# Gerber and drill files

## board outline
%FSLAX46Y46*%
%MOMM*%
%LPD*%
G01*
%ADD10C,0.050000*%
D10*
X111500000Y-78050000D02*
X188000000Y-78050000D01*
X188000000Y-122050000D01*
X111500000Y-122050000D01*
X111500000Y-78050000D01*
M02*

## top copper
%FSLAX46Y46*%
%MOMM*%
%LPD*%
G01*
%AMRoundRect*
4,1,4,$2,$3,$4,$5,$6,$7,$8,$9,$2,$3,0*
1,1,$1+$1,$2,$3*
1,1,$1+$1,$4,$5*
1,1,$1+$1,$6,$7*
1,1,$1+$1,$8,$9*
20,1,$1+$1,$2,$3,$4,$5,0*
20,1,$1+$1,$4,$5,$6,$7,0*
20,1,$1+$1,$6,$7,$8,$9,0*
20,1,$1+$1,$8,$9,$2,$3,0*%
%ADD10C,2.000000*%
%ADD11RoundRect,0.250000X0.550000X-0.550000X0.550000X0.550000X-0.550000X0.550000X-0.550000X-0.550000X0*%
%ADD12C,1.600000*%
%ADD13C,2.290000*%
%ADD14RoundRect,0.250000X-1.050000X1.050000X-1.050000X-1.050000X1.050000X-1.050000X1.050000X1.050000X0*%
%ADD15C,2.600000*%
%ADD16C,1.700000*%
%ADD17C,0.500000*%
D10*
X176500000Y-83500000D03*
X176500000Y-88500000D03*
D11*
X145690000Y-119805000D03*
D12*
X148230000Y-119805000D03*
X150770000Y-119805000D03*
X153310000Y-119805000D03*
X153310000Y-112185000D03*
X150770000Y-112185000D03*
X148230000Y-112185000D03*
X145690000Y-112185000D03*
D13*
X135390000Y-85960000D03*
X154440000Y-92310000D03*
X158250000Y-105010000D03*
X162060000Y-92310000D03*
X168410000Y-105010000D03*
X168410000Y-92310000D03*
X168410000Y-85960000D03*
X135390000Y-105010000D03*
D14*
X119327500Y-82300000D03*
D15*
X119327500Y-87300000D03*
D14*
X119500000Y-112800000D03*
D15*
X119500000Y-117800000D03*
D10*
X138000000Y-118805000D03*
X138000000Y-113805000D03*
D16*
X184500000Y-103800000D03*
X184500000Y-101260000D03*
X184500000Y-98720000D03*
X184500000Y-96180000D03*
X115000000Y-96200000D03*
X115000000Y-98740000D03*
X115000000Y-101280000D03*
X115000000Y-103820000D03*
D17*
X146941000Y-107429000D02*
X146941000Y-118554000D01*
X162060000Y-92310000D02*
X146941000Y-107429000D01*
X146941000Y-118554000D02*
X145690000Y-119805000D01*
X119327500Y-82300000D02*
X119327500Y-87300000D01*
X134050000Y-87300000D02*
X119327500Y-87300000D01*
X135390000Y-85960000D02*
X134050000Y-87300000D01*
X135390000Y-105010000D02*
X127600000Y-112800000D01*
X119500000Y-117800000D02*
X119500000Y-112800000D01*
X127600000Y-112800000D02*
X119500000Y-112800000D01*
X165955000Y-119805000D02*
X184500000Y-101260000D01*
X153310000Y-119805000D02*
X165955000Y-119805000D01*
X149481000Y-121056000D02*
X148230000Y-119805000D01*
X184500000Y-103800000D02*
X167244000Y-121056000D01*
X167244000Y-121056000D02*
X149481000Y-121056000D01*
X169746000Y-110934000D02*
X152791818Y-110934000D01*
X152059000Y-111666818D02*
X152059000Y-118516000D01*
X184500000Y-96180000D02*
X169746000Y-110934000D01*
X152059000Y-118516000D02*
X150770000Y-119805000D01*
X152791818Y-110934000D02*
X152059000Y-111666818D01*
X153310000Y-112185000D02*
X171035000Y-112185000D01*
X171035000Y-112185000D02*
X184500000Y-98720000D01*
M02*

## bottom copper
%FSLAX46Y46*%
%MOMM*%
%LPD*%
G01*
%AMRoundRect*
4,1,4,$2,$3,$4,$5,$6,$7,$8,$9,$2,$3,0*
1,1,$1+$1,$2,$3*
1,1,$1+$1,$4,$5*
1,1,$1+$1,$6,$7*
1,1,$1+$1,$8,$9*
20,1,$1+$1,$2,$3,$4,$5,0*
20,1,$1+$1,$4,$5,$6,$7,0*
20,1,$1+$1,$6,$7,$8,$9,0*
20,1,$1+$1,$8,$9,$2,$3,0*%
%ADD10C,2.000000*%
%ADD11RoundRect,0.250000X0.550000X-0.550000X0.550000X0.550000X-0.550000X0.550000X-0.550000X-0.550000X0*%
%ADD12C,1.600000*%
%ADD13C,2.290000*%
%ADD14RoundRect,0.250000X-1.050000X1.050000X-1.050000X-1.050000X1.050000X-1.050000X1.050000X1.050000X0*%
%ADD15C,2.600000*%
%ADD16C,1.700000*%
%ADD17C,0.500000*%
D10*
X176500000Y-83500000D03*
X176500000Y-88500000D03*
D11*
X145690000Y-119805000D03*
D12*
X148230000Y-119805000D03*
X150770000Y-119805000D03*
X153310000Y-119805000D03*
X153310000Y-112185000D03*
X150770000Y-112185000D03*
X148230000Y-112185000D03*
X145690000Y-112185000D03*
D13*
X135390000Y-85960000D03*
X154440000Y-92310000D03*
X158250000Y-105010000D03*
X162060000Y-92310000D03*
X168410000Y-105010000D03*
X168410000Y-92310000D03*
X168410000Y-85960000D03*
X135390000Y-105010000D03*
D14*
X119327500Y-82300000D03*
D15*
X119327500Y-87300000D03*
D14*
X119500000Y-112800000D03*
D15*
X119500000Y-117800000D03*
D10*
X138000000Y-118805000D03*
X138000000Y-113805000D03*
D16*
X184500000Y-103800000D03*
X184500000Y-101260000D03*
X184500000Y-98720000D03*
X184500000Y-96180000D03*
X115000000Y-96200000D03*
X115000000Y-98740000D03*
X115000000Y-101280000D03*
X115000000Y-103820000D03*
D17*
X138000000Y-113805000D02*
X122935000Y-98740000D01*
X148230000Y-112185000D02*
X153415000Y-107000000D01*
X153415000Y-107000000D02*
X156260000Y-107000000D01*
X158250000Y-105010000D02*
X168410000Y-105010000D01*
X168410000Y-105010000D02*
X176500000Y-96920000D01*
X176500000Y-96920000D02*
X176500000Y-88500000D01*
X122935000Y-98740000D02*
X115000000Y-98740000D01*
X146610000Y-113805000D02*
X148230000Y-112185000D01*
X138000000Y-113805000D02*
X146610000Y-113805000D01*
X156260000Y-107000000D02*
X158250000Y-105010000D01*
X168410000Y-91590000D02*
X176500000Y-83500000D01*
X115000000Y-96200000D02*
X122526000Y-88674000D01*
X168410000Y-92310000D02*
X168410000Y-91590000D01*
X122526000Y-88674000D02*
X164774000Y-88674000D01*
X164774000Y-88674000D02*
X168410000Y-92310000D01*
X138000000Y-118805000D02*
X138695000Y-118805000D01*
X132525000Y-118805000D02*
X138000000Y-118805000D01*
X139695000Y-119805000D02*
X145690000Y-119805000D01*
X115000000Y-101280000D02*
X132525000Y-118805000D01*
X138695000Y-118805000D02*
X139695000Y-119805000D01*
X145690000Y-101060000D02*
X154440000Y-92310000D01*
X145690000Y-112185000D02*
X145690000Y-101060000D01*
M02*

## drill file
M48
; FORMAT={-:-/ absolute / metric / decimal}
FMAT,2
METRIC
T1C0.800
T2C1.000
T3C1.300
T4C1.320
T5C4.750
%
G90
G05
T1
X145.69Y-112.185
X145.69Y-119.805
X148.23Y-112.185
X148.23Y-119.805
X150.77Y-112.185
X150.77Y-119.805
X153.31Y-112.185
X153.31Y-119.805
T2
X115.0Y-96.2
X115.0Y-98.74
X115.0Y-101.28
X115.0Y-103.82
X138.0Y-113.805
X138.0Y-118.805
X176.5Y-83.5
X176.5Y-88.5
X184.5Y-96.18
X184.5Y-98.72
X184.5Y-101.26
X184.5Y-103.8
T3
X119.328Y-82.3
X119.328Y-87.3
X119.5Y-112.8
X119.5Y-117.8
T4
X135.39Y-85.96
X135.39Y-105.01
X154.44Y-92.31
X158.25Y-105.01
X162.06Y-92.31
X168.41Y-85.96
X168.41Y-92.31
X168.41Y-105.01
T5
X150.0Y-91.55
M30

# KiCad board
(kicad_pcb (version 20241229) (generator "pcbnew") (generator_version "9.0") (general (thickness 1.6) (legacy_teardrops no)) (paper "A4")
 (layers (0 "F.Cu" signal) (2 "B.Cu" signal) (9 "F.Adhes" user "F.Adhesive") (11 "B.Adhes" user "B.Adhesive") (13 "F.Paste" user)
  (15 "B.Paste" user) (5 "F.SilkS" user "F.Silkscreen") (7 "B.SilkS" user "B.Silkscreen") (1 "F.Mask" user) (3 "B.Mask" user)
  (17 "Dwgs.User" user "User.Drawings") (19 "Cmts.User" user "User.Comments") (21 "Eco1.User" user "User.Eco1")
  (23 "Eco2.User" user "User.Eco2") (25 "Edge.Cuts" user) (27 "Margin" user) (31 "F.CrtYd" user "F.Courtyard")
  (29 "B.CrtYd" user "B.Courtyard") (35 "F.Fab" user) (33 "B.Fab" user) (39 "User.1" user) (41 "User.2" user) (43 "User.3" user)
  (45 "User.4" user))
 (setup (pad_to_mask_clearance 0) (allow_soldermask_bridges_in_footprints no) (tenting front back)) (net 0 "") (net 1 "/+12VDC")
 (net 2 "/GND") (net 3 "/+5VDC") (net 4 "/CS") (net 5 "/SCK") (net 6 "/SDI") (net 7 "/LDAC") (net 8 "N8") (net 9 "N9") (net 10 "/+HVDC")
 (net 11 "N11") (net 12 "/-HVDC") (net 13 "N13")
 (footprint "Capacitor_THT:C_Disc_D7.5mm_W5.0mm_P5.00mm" (layer "F.Cu") (at 176.5 83.5 -90)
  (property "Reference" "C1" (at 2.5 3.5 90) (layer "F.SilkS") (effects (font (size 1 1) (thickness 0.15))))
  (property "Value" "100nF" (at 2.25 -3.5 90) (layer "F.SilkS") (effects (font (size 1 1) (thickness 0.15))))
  (pad "1" thru_hole circle (at 0 0 270) (size 2 2) (drill 1) (layers "*.Cu" "*.Mask") (remove_unused_layers no) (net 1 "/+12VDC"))
  (pad "2" thru_hole circle (at 5 0 270) (size 2 2) (drill 1) (layers "*.Cu" "*.Mask") (remove_unused_layers no) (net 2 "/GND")))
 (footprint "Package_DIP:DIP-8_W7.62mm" (layer "F.Cu") (at 145.69 119.805 90)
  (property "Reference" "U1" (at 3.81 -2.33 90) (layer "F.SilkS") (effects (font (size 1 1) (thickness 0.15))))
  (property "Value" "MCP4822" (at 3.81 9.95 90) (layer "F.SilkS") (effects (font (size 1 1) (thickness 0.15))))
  (pad "1" thru_hole roundrect (at 0 0 90) (size 1.6 1.6) (drill 0.8) (layers "*.Cu" "*.Mask") (remove_unused_layers no)
   (roundrect_rratio 0.15625) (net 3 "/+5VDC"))
  (pad "2" thru_hole circle (at 0 2.54 90) (size 1.6 1.6) (drill 0.8) (layers "*.Cu" "*.Mask") (remove_unused_layers no) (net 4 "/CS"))
  (pad "3" thru_hole circle (at 0 5.08 90) (size 1.6 1.6) (drill 0.8) (layers "*.Cu" "*.Mask") (remove_unused_layers no) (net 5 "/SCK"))
  (pad "4" thru_hole circle (at 0 7.62 90) (size 1.6 1.6) (drill 0.8) (layers "*.Cu" "*.Mask") (remove_unused_layers no) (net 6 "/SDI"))
  (pad "5" thru_hole circle (at 7.62 7.62 90) (size 1.6 1.6) (drill 0.8) (layers "*.Cu" "*.Mask") (remove_unused_layers no) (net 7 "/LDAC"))
  (pad "6" thru_hole circle (at 7.62 5.08 90) (size 1.6 1.6) (drill 0.8) (layers "*.Cu" "*.Mask") (remove_unused_layers no) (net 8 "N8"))
  (pad "7" thru_hole circle (at 7.62 2.54 90) (size 1.6 1.6) (drill 0.8) (layers "*.Cu" "*.Mask") (remove_unused_layers no) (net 2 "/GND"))
  (pad "8" thru_hole circle (at 7.62 0 90) (size 1.6 1.6) (drill 0.8) (layers "*.Cu" "*.Mask") (remove_unused_layers no) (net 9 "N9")))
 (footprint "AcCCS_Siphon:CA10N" (layer "F.Cu") (at 135.39 85.96)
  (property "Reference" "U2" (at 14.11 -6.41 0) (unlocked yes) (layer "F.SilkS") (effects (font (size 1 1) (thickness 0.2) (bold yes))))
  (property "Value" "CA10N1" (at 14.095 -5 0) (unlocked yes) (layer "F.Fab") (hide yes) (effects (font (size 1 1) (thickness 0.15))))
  (pad "" np_thru_hole circle (at 14.61 5.59) (size 4.75 4.75) (drill 4.75) (layers "*.Cu" "*.Mask"))
  (pad "1" thru_hole circle (at 0 0) (size 2.29 2.29) (drill 1.32) (layers "*.Cu" "*.Mask") (remove_unused_layers no) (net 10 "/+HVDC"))
  (pad "2" thru_hole circle (at 19.05 6.35) (size 2.29 2.29) (drill 1.32) (layers "*.Cu" "*.Mask") (remove_unused_layers no) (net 9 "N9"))
  (pad "3" thru_hole circle (at 22.86 19.05) (size 2.29 2.29) (drill 1.32) (layers "*.Cu" "*.Mask") (remove_unused_layers no) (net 2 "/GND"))
  (pad "4" thru_hole circle (at 26.67 6.35) (size 2.29 2.29) (drill 1.32) (layers "*.Cu" "*.Mask") (remove_unused_layers no)
   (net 3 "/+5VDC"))
  (pad "5" thru_hole circle (at 33.02 19.05) (size 2.29 2.29) (drill 1.32) (layers "*.Cu" "*.Mask") (remove_unused_layers no) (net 2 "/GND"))
  (pad "6" thru_hole circle (at 33.02 6.35) (size 2.29 2.29) (drill 1.32) (layers "*.Cu" "*.Mask") (remove_unused_layers no)
   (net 1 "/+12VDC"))
  (pad "7" thru_hole circle (at 33.02 0) (size 2.29 2.29) (drill 1.32) (layers "*.Cu" "*.Mask") (remove_unused_layers no) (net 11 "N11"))
  (pad "8" thru_hole circle (at 0 19.05) (size 2.29 2.29) (drill 1.32) (layers "*.Cu" "*.Mask") (remove_unused_layers no) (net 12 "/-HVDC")))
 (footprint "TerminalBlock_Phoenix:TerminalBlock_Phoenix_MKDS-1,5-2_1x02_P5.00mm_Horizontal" (layer "F.Cu") (at 119.3275 82.3 -90)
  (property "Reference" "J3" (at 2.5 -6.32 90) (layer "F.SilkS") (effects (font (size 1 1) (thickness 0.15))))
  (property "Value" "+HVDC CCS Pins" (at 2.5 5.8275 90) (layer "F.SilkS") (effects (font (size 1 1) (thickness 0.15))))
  (pad "1" thru_hole roundrect (at 0 0 270) (size 2.6 2.6) (drill 1.3) (layers "*.Cu" "*.Mask") (remove_unused_layers no)
   (roundrect_rratio 0.096154) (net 10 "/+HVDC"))
  (pad "2" thru_hole circle (at 5 0 270) (size 2.6 2.6) (drill 1.3) (layers "*.Cu" "*.Mask") (remove_unused_layers no) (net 10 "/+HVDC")))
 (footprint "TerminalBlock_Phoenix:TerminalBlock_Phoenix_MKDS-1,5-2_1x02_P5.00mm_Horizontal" (layer "F.Cu") (at 119.5 112.8 -90)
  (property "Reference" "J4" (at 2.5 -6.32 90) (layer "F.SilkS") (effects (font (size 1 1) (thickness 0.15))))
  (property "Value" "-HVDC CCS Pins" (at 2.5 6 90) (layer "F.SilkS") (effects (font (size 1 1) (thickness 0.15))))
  (pad "1" thru_hole roundrect (at 0 0 270) (size 2.6 2.6) (drill 1.3) (layers "*.Cu" "*.Mask") (remove_unused_layers no)
   (roundrect_rratio 0.096154) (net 12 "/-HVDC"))
  (pad "2" thru_hole circle (at 5 0 270) (size 2.6 2.6) (drill 1.3) (layers "*.Cu" "*.Mask") (remove_unused_layers no) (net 12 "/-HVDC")))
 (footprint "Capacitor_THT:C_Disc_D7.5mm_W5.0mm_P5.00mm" (layer "F.Cu") (at 138 118.805 90)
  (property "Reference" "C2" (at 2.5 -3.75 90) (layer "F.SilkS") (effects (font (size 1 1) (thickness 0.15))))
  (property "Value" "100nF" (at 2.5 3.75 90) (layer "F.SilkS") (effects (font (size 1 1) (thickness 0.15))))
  (pad "1" thru_hole circle (at 0 0 90) (size 2 2) (drill 1) (layers "*.Cu" "*.Mask") (remove_unused_layers no) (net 3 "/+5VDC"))
  (pad "2" thru_hole circle (at 5 0 90) (size 2 2) (drill 1) (layers "*.Cu" "*.Mask") (remove_unused_layers no) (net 2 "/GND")))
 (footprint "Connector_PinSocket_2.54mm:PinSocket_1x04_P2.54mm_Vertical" (layer "B.Cu") (at 184.5 103.8)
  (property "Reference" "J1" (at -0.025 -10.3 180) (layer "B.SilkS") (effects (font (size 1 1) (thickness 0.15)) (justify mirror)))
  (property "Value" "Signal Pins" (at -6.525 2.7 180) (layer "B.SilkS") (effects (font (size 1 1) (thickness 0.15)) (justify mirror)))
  (pad "1" thru_hole circle (at 0 0) (size 1.7 1.7) (drill 1) (layers "*.Cu" "*.Mask") (remove_unused_layers no) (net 4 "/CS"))
  (pad "2" thru_hole circle (at 0 -2.54) (size 1.7 1.7) (drill 1) (layers "*.Cu" "*.Mask") (remove_unused_layers no) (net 6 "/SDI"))
  (pad "3" thru_hole circle (at 0 -5.08) (size 1.7 1.7) (drill 1) (layers "*.Cu" "*.Mask") (remove_unused_layers no) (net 7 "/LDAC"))
  (pad "4" thru_hole circle (at 0 -7.62) (size 1.7 1.7) (drill 1) (layers "*.Cu" "*.Mask") (remove_unused_layers no) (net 5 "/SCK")))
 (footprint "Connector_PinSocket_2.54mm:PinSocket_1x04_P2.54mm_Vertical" (layer "B.Cu") (at 115 96.2 180)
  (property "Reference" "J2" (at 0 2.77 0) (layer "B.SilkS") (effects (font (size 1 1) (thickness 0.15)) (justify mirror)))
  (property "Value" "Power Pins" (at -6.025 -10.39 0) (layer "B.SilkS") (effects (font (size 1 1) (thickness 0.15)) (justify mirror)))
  (pad "1" thru_hole circle (at 0 0 180) (size 1.7 1.7) (drill 1) (layers "*.Cu" "*.Mask") (remove_unused_layers no) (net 1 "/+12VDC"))
  (pad "2" thru_hole circle (at 0 -2.54 180) (size 1.7 1.7) (drill 1) (layers "*.Cu" "*.Mask") (remove_unused_layers no) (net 2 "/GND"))
  (pad "3" thru_hole circle (at 0 -5.08 180) (size 1.7 1.7) (drill 1) (layers "*.Cu" "*.Mask") (remove_unused_layers no) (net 3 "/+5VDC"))
  (pad "4" thru_hole circle (at 0 -7.62 180) (size 1.7 1.7) (drill 1) (layers "*.Cu" "*.Mask") (remove_unused_layers no) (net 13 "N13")))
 (gr_rect (start 111.5 78.05) (end 188 122.05) (stroke (width 0.05) (type default)) (fill no) (layer "Edge.Cuts"))
 (segment (start 138 113.805) (end 122.935 98.74) (width 0.5) (layer "B.Cu") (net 2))
 (segment (start 148.23 112.185) (end 153.415 107) (width 0.5) (layer "B.Cu") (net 2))
 (segment (start 153.415 107) (end 156.26 107) (width 0.5) (layer "B.Cu") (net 2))
 (segment (start 158.25 105.01) (end 168.41 105.01) (width 0.5) (layer "B.Cu") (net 2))
 (segment (start 168.41 105.01) (end 176.5 96.92) (width 0.5) (layer "B.Cu") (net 2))
 (segment (start 176.5 96.92) (end 176.5 88.5) (width 0.5) (layer "B.Cu") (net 2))
 (segment (start 122.935 98.74) (end 115 98.74) (width 0.5) (layer "B.Cu") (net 2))
 (segment (start 146.61 113.805) (end 148.23 112.185) (width 0.5) (layer "B.Cu") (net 2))
 (segment (start 138 113.805) (end 146.61 113.805) (width 0.5) (layer "B.Cu") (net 2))
 (segment (start 156.26 107) (end 158.25 105.01) (width 0.5) (layer "B.Cu") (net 2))
 (segment (start 168.41 91.59) (end 176.5 83.5) (width 0.5) (layer "B.Cu") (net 1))
 (segment (start 115 96.2) (end 122.526 88.674) (width 0.5) (layer "B.Cu") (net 1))
 (segment (start 168.41 92.31) (end 168.41 91.59) (width 0.5) (layer "B.Cu") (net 1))
 (segment (start 122.526 88.674) (end 164.774 88.674) (width 0.5) (layer "B.Cu") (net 1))
 (segment (start 164.774 88.674) (end 168.41 92.31) (width 0.5) (layer "B.Cu") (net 1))
 (segment (start 146.941 107.429) (end 146.941 118.554) (width 0.5) (layer "F.Cu") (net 3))
 (segment (start 162.06 92.31) (end 146.941 107.429) (width 0.5) (layer "F.Cu") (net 3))
 (segment (start 146.941 118.554) (end 145.69 119.805) (width 0.5) (layer "F.Cu") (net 3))
 (segment (start 138 118.805) (end 138.695 118.805) (width 0.5) (layer "B.Cu") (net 3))
 (segment (start 132.525 118.805) (end 138 118.805) (width 0.5) (layer "B.Cu") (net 3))
 (segment (start 139.695 119.805) (end 145.69 119.805) (width 0.5) (layer "B.Cu") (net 3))
 (segment (start 115 101.28) (end 132.525 118.805) (width 0.5) (layer "B.Cu") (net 3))
 (segment (start 138.695 118.805) (end 139.695 119.805) (width 0.5) (layer "B.Cu") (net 3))
 (segment (start 119.3275 82.3) (end 119.3275 87.3) (width 0.5) (layer "F.Cu") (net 10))
 (segment (start 134.05 87.3) (end 119.3275 87.3) (width 0.5) (layer "F.Cu") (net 10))
 (segment (start 135.39 85.96) (end 134.05 87.3) (width 0.5) (layer "F.Cu") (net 10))
 (segment (start 135.39 105.01) (end 127.6 112.8) (width 0.5) (layer "F.Cu") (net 12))
 (segment (start 119.5 117.8) (end 119.5 112.8) (width 0.5) (layer "F.Cu") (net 12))
 (segment (start 127.6 112.8) (end 119.5 112.8) (width 0.5) (layer "F.Cu") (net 12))
 (segment (start 165.955 119.805) (end 184.5 101.26) (width 0.5) (layer "F.Cu") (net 6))
 (segment (start 153.31 119.805) (end 165.955 119.805) (width 0.5) (layer "F.Cu") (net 6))
 (segment (start 149.481 121.056) (end 148.23 119.805) (width 0.5) (layer "F.Cu") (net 4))
 (segment (start 184.5 103.8) (end 167.244 121.056) (width 0.5) (layer "F.Cu") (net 4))
 (segment (start 167.244 121.056) (end 149.481 121.056) (width 0.5) (layer "F.Cu") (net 4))
 (segment (start 169.746 110.934) (end 152.791818 110.934) (width 0.5) (layer "F.Cu") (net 5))
 (segment (start 152.059 111.666818) (end 152.059 118.516) (width 0.5) (layer "F.Cu") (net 5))
 (segment (start 184.5 96.18) (end 169.746 110.934) (width 0.5) (layer "F.Cu") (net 5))
 (segment (start 152.059 118.516) (end 150.77 119.805) (width 0.5) (layer "F.Cu") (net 5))
 (segment (start 152.791818 110.934) (end 152.059 111.666818) (width 0.5) (layer "F.Cu") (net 5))
 (segment (start 153.31 112.185) (end 171.035 112.185) (width 0.5) (layer "F.Cu") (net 7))
 (segment (start 171.035 112.185) (end 184.5 98.72) (width 0.5) (layer "F.Cu") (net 7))
 (segment (start 145.69 101.06) (end 154.44 92.31) (width 0.5) (layer "B.Cu") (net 9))
 (segment (start 145.69 112.185) (end 145.69 101.06) (width 0.5) (layer "B.Cu") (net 9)))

